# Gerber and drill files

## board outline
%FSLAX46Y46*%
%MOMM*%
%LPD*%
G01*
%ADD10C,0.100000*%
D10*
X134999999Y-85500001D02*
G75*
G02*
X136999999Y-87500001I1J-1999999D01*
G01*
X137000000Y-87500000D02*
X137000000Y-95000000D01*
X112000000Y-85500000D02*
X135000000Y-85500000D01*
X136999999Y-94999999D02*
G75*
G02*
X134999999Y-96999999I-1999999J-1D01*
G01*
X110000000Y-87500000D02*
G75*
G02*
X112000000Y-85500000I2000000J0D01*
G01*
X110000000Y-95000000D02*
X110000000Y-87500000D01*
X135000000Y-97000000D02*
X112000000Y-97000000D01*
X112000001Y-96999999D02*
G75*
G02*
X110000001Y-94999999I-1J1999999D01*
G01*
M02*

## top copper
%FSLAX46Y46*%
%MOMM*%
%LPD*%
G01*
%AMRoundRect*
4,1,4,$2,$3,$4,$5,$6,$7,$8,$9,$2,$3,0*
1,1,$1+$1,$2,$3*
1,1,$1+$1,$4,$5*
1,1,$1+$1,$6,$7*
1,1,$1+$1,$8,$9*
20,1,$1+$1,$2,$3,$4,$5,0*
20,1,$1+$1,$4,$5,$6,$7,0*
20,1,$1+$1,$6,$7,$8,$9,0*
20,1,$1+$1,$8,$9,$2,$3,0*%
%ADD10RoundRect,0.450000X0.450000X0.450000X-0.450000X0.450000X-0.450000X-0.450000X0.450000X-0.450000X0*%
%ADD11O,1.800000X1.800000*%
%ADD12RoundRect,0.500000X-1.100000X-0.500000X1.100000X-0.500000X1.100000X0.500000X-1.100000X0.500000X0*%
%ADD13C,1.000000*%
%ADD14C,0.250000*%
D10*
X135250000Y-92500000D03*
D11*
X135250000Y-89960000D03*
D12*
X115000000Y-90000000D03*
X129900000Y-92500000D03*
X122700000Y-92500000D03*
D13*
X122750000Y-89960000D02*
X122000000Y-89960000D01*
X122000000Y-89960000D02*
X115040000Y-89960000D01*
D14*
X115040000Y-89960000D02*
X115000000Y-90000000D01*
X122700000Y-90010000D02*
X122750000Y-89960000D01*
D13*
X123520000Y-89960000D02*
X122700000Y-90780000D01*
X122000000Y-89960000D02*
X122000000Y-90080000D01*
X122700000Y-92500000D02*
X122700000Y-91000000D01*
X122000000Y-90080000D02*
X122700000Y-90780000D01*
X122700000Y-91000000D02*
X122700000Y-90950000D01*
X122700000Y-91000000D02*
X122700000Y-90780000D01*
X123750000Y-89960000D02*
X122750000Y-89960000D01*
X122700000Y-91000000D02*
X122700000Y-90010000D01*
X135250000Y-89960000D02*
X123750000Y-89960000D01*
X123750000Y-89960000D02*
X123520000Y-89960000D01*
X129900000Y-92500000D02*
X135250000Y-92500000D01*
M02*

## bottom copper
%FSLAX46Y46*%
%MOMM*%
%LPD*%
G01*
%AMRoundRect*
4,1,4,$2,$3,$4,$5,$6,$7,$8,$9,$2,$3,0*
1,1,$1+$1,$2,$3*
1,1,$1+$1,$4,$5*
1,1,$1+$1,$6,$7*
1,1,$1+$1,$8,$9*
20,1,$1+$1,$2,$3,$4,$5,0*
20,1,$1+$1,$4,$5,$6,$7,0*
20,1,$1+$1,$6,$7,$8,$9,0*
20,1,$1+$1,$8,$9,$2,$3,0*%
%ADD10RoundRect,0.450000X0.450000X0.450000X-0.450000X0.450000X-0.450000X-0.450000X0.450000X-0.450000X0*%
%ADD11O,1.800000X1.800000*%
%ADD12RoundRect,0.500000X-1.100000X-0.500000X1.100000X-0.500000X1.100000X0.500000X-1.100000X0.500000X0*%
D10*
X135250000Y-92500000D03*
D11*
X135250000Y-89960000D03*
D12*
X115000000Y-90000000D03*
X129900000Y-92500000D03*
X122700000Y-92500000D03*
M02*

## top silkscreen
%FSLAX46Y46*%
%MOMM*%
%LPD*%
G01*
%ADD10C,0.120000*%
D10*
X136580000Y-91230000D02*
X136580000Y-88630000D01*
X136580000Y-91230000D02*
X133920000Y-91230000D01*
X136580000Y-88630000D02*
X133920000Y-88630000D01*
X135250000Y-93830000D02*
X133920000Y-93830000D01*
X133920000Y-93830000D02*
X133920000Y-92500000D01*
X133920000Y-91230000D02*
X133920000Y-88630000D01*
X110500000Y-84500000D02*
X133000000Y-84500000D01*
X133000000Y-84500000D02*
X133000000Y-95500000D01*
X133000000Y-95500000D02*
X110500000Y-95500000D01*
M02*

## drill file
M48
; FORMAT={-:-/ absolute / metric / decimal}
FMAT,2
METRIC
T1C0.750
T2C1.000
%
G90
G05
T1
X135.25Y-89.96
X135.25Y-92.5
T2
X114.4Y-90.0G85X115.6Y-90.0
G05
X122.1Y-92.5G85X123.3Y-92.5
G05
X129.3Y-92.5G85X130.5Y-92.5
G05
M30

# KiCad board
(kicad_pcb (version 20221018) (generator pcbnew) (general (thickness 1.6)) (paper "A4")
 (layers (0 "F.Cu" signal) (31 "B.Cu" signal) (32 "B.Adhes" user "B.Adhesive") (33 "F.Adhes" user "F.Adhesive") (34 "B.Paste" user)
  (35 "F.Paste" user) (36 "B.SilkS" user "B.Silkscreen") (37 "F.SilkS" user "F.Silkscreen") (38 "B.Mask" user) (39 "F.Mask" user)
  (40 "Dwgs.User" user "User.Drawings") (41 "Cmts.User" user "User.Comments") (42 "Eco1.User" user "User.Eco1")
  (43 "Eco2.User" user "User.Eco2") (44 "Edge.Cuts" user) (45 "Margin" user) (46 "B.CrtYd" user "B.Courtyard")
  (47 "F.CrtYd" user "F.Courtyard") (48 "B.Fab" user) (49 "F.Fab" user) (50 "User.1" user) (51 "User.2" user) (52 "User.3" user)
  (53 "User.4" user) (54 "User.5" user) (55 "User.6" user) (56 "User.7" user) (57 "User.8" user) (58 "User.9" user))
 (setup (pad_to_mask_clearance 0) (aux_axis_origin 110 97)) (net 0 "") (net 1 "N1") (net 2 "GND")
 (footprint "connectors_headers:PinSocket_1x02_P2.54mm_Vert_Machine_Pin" (layer "F.Cu") (at 135.25 92.5 180)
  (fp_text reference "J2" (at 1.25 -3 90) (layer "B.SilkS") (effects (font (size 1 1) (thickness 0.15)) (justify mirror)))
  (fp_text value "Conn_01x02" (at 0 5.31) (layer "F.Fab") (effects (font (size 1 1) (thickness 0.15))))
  (fp_line (start -1.33 1.27) (end -1.33 3.87) (stroke (width 0.12) (type solid)) (layer "F.SilkS"))
  (fp_line (start -1.33 1.27) (end 1.33 1.27) (stroke (width 0.12) (type solid)) (layer "F.SilkS"))
  (fp_line (start -1.33 3.87) (end 1.33 3.87) (stroke (width 0.12) (type solid)) (layer "F.SilkS"))
  (fp_line (start 0 -1.33) (end 1.33 -1.33) (stroke (width 0.12) (type solid)) (layer "F.SilkS"))
  (fp_line (start 1.33 -1.33) (end 1.33 0) (stroke (width 0.12) (type solid)) (layer "F.SilkS"))
  (fp_line (start 1.33 1.27) (end 1.33 3.87) (stroke (width 0.12) (type solid)) (layer "F.SilkS"))
  (pad "1" thru_hole roundrect (at 0 0 180) (size 1.8 1.8) (drill 0.75) (layers "*.Cu" "*.Mask") (roundrect_rratio 0.25) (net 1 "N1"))
  (pad "2" thru_hole oval (at 0 2.54 180) (size 1.8 1.8) (drill 0.75) (layers "*.Cu" "*.Mask") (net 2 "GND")))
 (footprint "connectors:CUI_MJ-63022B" (layer "F.Cu") (at 107.5 90)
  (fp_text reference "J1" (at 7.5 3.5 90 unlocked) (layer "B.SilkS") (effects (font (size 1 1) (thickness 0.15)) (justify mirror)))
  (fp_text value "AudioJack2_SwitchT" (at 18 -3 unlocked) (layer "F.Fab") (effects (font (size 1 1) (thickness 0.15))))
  (fp_line (start 3 -5.5) (end 25.5 -5.5) (stroke (width 0.12) (type default)) (layer "F.SilkS"))
  (fp_line (start 25.5 -5.5) (end 25.5 5.5) (stroke (width 0.12) (type default)) (layer "F.SilkS"))
  (fp_line (start 25.5 5.5) (end 3 5.5) (stroke (width 0.12) (type default)) (layer "F.SilkS"))
  (pad "1" thru_hole roundrect (at 7.5 0) (size 3.2 2) (drill oval 2.2 1) (layers "*.Cu" "*.Mask") (roundrect_rratio 0.25) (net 2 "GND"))
  (pad "2" thru_hole roundrect (at 22.4 2.5) (size 3.2 2) (drill oval 2.2 1) (layers "*.Cu" "*.Mask") (roundrect_rratio 0.25) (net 1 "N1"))
  (pad "3" thru_hole roundrect (at 15.2 2.5) (size 3.2 2) (drill oval 2.2 1) (layers "*.Cu" "*.Mask") (roundrect_rratio 0.25) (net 2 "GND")))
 (gr_arc (start 134.999999 85.500001) (mid 136.414213 86.085787) (end 136.999999 87.500001) (stroke (width 0.1) (type default))
  (layer "Edge.Cuts"))
 (gr_line (start 137 87.5) (end 137 95) (stroke (width 0.1) (type default)) (layer "Edge.Cuts"))
 (gr_line (start 112 85.5) (end 135 85.5) (stroke (width 0.1) (type default)) (layer "Edge.Cuts"))
 (gr_arc (start 136.999999 94.999999) (mid 136.414213 96.414213) (end 134.999999 96.999999) (stroke (width 0.1) (type default))
  (layer "Edge.Cuts"))
 (gr_arc (start 110 87.5) (mid 110.585786 86.085786) (end 112 85.5) (stroke (width 0.1) (type default)) (layer "Edge.Cuts"))
 (gr_line (start 110 95) (end 110 87.5) (stroke (width 0.1) (type default)) (layer "Edge.Cuts"))
 (gr_line (start 135 97) (end 112 97) (stroke (width 0.1) (type default)) (layer "Edge.Cuts"))
 (gr_arc (start 112.000001 96.999999) (mid 110.585787 96.414213) (end 110.000001 94.999999) (stroke (width 0.1) (type default))
  (layer "Edge.Cuts"))
 (segment (start 122.75 89.96) (end 122 89.96) (width 1) (layer "F.Cu") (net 2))
 (segment (start 122 89.96) (end 115.04 89.96) (width 1) (layer "F.Cu") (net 2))
 (segment (start 115.04 89.96) (end 115 90) (width 0.25) (layer "F.Cu") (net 2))
 (segment (start 122.7 90.01) (end 122.75 89.96) (width 0.25) (layer "F.Cu") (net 2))
 (segment (start 123.52 89.96) (end 122.7 90.78) (width 1) (layer "F.Cu") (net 2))
 (segment (start 122 89.96) (end 122 90.08) (width 1) (layer "F.Cu") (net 2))
 (segment (start 122.7 92.5) (end 122.7 91) (width 1) (layer "F.Cu") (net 2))
 (segment (start 122 90.08) (end 122.7 90.78) (width 1) (layer "F.Cu") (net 2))
 (segment (start 122.7 91) (end 122.7 90.95) (width 1) (layer "F.Cu") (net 2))
 (segment (start 122.7 91) (end 122.7 90.78) (width 1) (layer "F.Cu") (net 2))
 (segment (start 123.75 89.96) (end 122.75 89.96) (width 1) (layer "F.Cu") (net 2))
 (segment (start 122.7 91) (end 122.7 90.01) (width 1) (layer "F.Cu") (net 2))
 (segment (start 135.25 89.96) (end 123.75 89.96) (width 1) (layer "F.Cu") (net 2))
 (segment (start 123.75 89.96) (end 123.52 89.96) (width 1) (layer "F.Cu") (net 2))
 (segment (start 129.9 92.5) (end 135.25 92.5) (width 1) (layer "F.Cu") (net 1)))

